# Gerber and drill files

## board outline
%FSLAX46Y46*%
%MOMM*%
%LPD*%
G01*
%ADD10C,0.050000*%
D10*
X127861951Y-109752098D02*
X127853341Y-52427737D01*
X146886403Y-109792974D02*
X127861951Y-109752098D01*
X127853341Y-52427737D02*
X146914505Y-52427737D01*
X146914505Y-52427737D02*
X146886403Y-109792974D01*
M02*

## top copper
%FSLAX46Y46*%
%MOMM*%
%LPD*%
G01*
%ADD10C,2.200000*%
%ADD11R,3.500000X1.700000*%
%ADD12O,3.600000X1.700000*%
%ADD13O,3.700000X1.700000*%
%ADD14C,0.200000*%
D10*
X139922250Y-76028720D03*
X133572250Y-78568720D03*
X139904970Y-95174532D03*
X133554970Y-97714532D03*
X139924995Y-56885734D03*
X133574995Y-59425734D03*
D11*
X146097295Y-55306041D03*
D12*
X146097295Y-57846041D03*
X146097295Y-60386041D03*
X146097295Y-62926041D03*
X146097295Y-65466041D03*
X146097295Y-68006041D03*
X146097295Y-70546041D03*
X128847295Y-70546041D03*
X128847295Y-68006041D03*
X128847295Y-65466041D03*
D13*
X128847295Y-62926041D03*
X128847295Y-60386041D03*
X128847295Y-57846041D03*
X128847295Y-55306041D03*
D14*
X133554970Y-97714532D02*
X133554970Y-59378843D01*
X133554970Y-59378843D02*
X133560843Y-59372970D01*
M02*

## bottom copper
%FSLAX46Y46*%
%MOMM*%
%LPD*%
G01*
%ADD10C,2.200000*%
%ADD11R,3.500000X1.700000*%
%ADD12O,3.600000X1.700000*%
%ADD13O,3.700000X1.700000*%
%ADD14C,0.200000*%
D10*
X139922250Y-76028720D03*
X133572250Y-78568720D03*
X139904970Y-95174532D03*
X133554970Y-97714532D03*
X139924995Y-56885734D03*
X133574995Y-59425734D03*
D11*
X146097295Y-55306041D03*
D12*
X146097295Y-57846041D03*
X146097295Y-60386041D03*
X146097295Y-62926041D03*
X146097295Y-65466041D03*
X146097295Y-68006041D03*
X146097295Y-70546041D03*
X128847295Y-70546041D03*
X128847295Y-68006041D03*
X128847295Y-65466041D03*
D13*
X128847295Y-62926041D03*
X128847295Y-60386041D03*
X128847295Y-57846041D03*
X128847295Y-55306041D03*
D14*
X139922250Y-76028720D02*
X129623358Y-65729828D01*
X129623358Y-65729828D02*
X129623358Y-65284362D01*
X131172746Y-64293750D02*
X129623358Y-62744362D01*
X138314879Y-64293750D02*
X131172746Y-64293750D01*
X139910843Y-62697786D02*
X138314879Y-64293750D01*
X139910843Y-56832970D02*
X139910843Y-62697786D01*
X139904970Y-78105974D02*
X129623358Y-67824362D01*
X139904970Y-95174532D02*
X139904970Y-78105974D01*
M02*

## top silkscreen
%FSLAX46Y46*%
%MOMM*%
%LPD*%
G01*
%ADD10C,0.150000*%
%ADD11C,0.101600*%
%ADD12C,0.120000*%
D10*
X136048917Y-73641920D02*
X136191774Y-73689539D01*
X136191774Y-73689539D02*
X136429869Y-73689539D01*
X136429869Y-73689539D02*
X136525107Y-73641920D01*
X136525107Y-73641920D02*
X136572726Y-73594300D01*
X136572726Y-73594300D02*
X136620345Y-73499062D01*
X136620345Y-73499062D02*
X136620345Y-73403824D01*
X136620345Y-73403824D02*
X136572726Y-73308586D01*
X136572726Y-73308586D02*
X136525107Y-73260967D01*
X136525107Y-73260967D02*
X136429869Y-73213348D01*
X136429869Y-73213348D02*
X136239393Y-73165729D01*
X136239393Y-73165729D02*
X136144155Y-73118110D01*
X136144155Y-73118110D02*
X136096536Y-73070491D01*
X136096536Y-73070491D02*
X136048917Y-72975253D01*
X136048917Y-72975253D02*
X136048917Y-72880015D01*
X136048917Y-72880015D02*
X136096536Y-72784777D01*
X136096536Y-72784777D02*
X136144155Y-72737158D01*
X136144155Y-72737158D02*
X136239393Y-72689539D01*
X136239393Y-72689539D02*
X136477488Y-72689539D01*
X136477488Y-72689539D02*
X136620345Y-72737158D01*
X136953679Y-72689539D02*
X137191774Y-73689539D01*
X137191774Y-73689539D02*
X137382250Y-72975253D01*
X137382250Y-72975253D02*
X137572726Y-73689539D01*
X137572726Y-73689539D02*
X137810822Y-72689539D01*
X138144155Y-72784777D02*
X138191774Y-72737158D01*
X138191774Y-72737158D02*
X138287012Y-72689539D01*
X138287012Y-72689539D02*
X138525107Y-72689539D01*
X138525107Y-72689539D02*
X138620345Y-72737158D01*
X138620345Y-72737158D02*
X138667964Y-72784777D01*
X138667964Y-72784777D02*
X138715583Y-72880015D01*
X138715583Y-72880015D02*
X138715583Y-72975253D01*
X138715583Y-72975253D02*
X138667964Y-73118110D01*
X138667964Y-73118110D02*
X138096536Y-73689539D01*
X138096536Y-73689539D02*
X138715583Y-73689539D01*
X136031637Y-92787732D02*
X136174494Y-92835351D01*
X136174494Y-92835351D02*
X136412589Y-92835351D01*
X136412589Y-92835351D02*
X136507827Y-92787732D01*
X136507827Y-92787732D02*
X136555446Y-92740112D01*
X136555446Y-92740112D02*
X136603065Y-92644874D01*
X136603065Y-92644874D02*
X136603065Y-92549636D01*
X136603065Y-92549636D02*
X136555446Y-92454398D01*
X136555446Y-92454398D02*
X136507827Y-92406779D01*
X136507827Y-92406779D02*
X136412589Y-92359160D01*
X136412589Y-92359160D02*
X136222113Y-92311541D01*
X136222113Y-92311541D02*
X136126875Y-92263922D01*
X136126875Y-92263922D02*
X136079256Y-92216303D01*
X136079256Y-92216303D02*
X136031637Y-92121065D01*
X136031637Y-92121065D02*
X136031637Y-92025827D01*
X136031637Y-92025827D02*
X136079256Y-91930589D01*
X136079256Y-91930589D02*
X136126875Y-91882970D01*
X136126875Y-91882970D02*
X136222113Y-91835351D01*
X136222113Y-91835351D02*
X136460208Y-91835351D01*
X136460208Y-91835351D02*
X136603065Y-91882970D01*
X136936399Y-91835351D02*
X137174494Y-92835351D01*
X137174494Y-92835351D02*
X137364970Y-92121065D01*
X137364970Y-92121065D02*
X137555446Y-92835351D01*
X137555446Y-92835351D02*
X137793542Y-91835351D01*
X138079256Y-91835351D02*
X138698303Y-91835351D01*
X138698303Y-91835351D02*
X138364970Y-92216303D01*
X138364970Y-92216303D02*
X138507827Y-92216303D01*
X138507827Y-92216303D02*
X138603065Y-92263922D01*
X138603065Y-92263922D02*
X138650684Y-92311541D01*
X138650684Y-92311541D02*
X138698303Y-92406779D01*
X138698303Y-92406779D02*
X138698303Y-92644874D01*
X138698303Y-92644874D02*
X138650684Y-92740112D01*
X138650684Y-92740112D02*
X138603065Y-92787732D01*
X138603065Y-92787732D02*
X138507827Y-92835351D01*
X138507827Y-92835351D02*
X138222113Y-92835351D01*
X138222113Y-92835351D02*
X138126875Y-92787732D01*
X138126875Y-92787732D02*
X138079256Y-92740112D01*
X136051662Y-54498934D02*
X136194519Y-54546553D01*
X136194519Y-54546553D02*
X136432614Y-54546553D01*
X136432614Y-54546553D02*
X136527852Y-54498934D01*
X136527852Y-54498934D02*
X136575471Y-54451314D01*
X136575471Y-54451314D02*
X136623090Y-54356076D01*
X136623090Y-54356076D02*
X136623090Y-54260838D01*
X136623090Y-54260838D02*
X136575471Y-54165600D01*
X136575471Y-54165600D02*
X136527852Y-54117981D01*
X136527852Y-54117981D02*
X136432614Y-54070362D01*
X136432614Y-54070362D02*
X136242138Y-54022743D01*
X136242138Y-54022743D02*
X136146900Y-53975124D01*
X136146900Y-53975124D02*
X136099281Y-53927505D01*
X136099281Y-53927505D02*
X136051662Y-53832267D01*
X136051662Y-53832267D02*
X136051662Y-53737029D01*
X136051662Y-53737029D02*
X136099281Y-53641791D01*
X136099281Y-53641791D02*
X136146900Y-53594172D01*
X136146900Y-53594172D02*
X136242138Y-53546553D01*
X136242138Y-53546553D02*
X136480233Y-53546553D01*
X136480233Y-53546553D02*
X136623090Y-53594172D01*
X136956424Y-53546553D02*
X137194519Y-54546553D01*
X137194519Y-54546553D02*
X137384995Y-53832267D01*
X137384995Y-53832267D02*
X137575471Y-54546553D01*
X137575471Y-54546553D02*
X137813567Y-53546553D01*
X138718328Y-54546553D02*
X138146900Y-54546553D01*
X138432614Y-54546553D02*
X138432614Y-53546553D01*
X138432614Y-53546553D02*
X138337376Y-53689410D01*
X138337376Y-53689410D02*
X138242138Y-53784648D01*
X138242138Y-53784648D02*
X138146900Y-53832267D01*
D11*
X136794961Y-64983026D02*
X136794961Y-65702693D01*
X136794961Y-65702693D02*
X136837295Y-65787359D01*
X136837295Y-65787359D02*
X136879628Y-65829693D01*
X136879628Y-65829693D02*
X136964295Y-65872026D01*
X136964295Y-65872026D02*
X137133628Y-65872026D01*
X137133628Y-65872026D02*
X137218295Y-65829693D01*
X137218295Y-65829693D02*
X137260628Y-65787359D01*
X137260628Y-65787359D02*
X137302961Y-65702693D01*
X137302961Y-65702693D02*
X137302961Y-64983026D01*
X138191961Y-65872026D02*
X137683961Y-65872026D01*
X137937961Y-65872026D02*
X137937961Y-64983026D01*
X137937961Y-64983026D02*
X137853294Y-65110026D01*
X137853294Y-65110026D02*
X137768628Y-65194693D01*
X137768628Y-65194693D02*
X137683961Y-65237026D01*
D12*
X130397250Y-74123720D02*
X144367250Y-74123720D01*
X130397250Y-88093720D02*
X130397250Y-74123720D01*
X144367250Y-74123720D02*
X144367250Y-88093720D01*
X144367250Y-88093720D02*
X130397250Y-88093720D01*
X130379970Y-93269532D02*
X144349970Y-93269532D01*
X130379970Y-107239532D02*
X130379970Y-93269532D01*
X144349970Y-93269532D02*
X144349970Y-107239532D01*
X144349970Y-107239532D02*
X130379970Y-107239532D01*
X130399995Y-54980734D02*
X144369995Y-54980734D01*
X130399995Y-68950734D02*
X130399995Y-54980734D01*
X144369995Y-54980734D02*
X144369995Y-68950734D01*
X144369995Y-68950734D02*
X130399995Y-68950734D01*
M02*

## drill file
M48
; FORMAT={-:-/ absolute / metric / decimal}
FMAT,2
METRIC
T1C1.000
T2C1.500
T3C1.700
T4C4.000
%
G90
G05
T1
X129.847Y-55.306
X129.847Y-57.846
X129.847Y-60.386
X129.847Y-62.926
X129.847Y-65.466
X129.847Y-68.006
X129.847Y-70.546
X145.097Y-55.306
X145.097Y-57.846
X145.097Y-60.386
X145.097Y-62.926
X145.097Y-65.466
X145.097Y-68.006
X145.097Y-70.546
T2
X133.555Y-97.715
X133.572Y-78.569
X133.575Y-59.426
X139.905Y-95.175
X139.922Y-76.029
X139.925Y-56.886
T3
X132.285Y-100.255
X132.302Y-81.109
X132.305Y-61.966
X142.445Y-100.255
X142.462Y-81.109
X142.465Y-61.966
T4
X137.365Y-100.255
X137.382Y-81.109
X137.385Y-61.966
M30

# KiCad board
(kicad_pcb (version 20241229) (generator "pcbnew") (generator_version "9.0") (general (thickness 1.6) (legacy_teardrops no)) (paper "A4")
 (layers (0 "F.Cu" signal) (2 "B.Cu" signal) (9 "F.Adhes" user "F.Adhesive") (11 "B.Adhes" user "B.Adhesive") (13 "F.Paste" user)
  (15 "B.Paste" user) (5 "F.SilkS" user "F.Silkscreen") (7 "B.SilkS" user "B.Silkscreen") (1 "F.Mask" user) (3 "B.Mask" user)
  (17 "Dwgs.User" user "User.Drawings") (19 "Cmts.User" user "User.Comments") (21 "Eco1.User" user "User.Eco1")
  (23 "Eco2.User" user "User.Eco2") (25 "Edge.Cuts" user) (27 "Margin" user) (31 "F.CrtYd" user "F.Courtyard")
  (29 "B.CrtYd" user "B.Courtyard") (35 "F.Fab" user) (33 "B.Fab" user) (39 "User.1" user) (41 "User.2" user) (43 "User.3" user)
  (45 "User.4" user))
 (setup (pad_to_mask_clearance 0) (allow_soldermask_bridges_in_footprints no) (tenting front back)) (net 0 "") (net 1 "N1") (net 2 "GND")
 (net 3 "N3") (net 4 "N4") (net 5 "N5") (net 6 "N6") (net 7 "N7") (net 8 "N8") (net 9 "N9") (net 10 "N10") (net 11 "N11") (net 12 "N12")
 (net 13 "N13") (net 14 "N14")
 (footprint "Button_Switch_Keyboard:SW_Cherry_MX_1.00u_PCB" (layer "F.Cu") (at 139.92225 76.02872)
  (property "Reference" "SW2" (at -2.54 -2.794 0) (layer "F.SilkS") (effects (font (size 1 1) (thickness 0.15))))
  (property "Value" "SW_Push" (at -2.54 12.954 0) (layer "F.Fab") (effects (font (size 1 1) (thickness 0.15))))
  (fp_line (start -9.525 -1.905) (end 4.445 -1.905) (stroke (width 0.12) (type solid)) (layer "F.SilkS"))
  (fp_line (start -9.525 12.065) (end -9.525 -1.905) (stroke (width 0.12) (type solid)) (layer "F.SilkS"))
  (fp_line (start 4.445 -1.905) (end 4.445 12.065) (stroke (width 0.12) (type solid)) (layer "F.SilkS"))
  (fp_line (start 4.445 12.065) (end -9.525 12.065) (stroke (width 0.12) (type solid)) (layer "F.SilkS"))
  (pad "" np_thru_hole circle (at -7.62 5.08) (size 1.7 1.7) (drill 1.7) (layers "*.Cu" "*.Mask"))
  (pad "" np_thru_hole circle (at -2.54 5.08) (size 4 4) (drill 4) (layers "*.Cu" "*.Mask"))
  (pad "" np_thru_hole circle (at 2.54 5.08) (size 1.7 1.7) (drill 1.7) (layers "*.Cu" "*.Mask"))
  (pad "1" thru_hole circle (at 0 0) (size 2.2 2.2) (drill 1.5) (layers "*.Cu" "*.Mask") (remove_unused_layers no) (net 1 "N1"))
  (pad "2" thru_hole circle (at -6.35 2.54) (size 2.2 2.2) (drill 1.5) (layers "*.Cu" "*.Mask") (remove_unused_layers no) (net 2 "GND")))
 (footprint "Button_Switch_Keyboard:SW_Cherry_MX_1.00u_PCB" (layer "F.Cu") (at 139.90497 95.174532)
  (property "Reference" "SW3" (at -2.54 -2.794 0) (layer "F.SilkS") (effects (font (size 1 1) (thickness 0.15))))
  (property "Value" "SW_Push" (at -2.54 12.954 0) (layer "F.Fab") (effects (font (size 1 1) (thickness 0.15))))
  (fp_line (start -9.525 -1.905) (end 4.445 -1.905) (stroke (width 0.12) (type solid)) (layer "F.SilkS"))
  (fp_line (start -9.525 12.065) (end -9.525 -1.905) (stroke (width 0.12) (type solid)) (layer "F.SilkS"))
  (fp_line (start 4.445 -1.905) (end 4.445 12.065) (stroke (width 0.12) (type solid)) (layer "F.SilkS"))
  (fp_line (start 4.445 12.065) (end -9.525 12.065) (stroke (width 0.12) (type solid)) (layer "F.SilkS"))
  (pad "" np_thru_hole circle (at -7.62 5.08) (size 1.7 1.7) (drill 1.7) (layers "*.Cu" "*.Mask"))
  (pad "" np_thru_hole circle (at -2.54 5.08) (size 4 4) (drill 4) (layers "*.Cu" "*.Mask"))
  (pad "" np_thru_hole circle (at 2.54 5.08) (size 1.7 1.7) (drill 1.7) (layers "*.Cu" "*.Mask"))
  (pad "1" thru_hole circle (at 0 0) (size 2.2 2.2) (drill 1.5) (layers "*.Cu" "*.Mask") (remove_unused_layers no) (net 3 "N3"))
  (pad "2" thru_hole circle (at -6.35 2.54) (size 2.2 2.2) (drill 1.5) (layers "*.Cu" "*.Mask") (remove_unused_layers no) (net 2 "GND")))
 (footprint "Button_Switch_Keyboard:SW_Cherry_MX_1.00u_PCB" (layer "F.Cu") (at 139.924995 56.885734)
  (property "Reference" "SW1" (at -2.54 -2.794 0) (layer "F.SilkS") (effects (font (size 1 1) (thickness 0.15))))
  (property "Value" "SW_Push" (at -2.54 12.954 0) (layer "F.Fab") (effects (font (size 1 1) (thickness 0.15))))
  (fp_line (start -9.525 -1.905) (end 4.445 -1.905) (stroke (width 0.12) (type solid)) (layer "F.SilkS"))
  (fp_line (start -9.525 12.065) (end -9.525 -1.905) (stroke (width 0.12) (type solid)) (layer "F.SilkS"))
  (fp_line (start 4.445 -1.905) (end 4.445 12.065) (stroke (width 0.12) (type solid)) (layer "F.SilkS"))
  (fp_line (start 4.445 12.065) (end -9.525 12.065) (stroke (width 0.12) (type solid)) (layer "F.SilkS"))
  (pad "" np_thru_hole circle (at -7.62 5.08) (size 1.7 1.7) (drill 1.7) (layers "*.Cu" "*.Mask"))
  (pad "" np_thru_hole circle (at -2.54 5.08) (size 4 4) (drill 4) (layers "*.Cu" "*.Mask"))
  (pad "" np_thru_hole circle (at 2.54 5.08) (size 1.7 1.7) (drill 1.7) (layers "*.Cu" "*.Mask"))
  (pad "1" thru_hole circle (at 0 0) (size 2.2 2.2) (drill 1.5) (layers "*.Cu" "*.Mask") (remove_unused_layers no) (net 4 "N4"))
  (pad "2" thru_hole circle (at -6.35 2.54) (size 2.2 2.2) (drill 1.5) (layers "*.Cu" "*.Mask") (remove_unused_layers no) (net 2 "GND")))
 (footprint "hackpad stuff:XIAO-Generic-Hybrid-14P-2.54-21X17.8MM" (layer "B.Cu") (at 137.472295 62.926041 180)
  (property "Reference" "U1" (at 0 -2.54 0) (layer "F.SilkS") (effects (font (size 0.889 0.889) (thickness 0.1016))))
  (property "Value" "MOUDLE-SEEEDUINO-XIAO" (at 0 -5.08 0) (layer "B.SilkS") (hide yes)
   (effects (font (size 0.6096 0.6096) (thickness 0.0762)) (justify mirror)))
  (pad "1" thru_hole rect (at -7.625 7.62 180) (size 3.5 1.7) (drill 1 (offset -1 0)) (layers "*.Cu" "*.Mask") (remove_unused_layers no)
   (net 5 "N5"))
  (pad "2" thru_hole oval (at -7.625 5.08 180) (size 3.6 1.7) (drill 1 (offset -1 0)) (layers "*.Cu" "*.Mask") (remove_unused_layers no)
   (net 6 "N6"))
  (pad "3" thru_hole oval (at -7.625 2.54 180) (size 3.6 1.7) (drill 1 (offset -1 0)) (layers "*.Cu" "*.Mask") (remove_unused_layers no)
   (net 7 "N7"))
  (pad "4" thru_hole oval (at -7.625 0 180) (size 3.6 1.7) (drill 1 (offset -1 0)) (layers "*.Cu" "*.Mask") (remove_unused_layers no)
   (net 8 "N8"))
  (pad "5" thru_hole oval (at -7.625 -2.54 180) (size 3.6 1.7) (drill 1 (offset -1 0)) (layers "*.Cu" "*.Mask") (remove_unused_layers no)
   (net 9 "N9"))
  (pad "6" thru_hole oval (at -7.625 -5.08) (size 3.6 1.7) (drill 1 (offset 1 0)) (layers "*.Cu" "*.Mask") (remove_unused_layers no)
   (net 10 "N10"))
  (pad "7" thru_hole oval (at -7.625 -7.62 180) (size 3.6 1.7) (drill 1 (offset -1 0)) (layers "*.Cu" "*.Mask") (remove_unused_layers no)
   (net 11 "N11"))
  (pad "8" thru_hole oval (at 7.625 -7.62 180) (size 3.6 1.7) (drill 1 (offset 1 0)) (layers "*.Cu" "*.Mask") (remove_unused_layers no)
   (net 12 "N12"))
  (pad "9" thru_hole oval (at 7.625 -5.08 180) (size 3.6 1.7) (drill 1 (offset 1 0)) (layers "*.Cu" "*.Mask") (remove_unused_layers no)
   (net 3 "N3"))
  (pad "10" thru_hole oval (at 7.625 -2.54 180) (size 3.6 1.7) (drill 1 (offset 1 0)) (layers "*.Cu" "*.Mask") (remove_unused_layers no)
   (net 1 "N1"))
  (pad "11" thru_hole oval (at 7.625 0 180) (size 3.7 1.7) (drill 1 (offset 1 0)) (layers "*.Cu" "*.Mask") (remove_unused_layers no)
   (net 4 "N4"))
  (pad "12" thru_hole oval (at 7.625 2.54 180) (size 3.7 1.7) (drill 1 (offset 1 0)) (layers "*.Cu" "*.Mask") (remove_unused_layers no)
   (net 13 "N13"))
  (pad "13" thru_hole oval (at 7.625 5.08 180) (size 3.7 1.7) (drill 1 (offset 1 0)) (layers "*.Cu" "*.Mask") (remove_unused_layers no)
   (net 2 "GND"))
  (pad "14" thru_hole oval (at 7.625 7.62 180) (size 3.7 1.7) (drill 1 (offset 1 0)) (layers "*.Cu" "*.Mask") (remove_unused_layers no)
   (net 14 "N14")))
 (gr_line (start 127.861951 109.752098) (end 127.853341 52.427737) (stroke (width 0.05) (type default)) (layer "Edge.Cuts"))
 (gr_line (start 146.886403 109.792974) (end 127.861951 109.752098) (stroke (width 0.05) (type default)) (layer "Edge.Cuts"))
 (gr_line (start 127.853341 52.427737) (end 146.914505 52.427737) (stroke (width 0.05) (type default)) (layer "Edge.Cuts"))
 (gr_line (start 146.914505 52.427737) (end 146.886403 109.792974) (stroke (width 0.05) (type default)) (layer "Edge.Cuts"))
 (segment (start 139.92225 76.02872) (end 129.623358 65.729828) (width 0.2) (layer "B.Cu") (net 1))
 (segment (start 129.623358 65.729828) (end 129.623358 65.284362) (width 0.2) (layer "B.Cu") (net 1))
 (segment (start 131.172746 64.29375) (end 129.623358 62.744362) (width 0.2) (layer "B.Cu") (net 4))
 (segment (start 138.314879 64.29375) (end 131.172746 64.29375) (width 0.2) (layer "B.Cu") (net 4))
 (segment (start 139.910843 62.697786) (end 138.314879 64.29375) (width 0.2) (layer "B.Cu") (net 4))
 (segment (start 139.910843 56.83297) (end 139.910843 62.697786) (width 0.2) (layer "B.Cu") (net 4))
 (segment (start 139.90497 78.105974) (end 129.623358 67.824362) (width 0.2) (layer "B.Cu") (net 3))
 (segment (start 139.90497 95.174532) (end 139.90497 78.105974) (width 0.2) (layer "B.Cu") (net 3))
 (segment (start 133.55497 97.714532) (end 133.55497 59.378843) (width 0.2) (layer "F.Cu") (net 2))
 (segment (start 133.55497 59.378843) (end 133.560843 59.37297) (width 0.2) (layer "F.Cu") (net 2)))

